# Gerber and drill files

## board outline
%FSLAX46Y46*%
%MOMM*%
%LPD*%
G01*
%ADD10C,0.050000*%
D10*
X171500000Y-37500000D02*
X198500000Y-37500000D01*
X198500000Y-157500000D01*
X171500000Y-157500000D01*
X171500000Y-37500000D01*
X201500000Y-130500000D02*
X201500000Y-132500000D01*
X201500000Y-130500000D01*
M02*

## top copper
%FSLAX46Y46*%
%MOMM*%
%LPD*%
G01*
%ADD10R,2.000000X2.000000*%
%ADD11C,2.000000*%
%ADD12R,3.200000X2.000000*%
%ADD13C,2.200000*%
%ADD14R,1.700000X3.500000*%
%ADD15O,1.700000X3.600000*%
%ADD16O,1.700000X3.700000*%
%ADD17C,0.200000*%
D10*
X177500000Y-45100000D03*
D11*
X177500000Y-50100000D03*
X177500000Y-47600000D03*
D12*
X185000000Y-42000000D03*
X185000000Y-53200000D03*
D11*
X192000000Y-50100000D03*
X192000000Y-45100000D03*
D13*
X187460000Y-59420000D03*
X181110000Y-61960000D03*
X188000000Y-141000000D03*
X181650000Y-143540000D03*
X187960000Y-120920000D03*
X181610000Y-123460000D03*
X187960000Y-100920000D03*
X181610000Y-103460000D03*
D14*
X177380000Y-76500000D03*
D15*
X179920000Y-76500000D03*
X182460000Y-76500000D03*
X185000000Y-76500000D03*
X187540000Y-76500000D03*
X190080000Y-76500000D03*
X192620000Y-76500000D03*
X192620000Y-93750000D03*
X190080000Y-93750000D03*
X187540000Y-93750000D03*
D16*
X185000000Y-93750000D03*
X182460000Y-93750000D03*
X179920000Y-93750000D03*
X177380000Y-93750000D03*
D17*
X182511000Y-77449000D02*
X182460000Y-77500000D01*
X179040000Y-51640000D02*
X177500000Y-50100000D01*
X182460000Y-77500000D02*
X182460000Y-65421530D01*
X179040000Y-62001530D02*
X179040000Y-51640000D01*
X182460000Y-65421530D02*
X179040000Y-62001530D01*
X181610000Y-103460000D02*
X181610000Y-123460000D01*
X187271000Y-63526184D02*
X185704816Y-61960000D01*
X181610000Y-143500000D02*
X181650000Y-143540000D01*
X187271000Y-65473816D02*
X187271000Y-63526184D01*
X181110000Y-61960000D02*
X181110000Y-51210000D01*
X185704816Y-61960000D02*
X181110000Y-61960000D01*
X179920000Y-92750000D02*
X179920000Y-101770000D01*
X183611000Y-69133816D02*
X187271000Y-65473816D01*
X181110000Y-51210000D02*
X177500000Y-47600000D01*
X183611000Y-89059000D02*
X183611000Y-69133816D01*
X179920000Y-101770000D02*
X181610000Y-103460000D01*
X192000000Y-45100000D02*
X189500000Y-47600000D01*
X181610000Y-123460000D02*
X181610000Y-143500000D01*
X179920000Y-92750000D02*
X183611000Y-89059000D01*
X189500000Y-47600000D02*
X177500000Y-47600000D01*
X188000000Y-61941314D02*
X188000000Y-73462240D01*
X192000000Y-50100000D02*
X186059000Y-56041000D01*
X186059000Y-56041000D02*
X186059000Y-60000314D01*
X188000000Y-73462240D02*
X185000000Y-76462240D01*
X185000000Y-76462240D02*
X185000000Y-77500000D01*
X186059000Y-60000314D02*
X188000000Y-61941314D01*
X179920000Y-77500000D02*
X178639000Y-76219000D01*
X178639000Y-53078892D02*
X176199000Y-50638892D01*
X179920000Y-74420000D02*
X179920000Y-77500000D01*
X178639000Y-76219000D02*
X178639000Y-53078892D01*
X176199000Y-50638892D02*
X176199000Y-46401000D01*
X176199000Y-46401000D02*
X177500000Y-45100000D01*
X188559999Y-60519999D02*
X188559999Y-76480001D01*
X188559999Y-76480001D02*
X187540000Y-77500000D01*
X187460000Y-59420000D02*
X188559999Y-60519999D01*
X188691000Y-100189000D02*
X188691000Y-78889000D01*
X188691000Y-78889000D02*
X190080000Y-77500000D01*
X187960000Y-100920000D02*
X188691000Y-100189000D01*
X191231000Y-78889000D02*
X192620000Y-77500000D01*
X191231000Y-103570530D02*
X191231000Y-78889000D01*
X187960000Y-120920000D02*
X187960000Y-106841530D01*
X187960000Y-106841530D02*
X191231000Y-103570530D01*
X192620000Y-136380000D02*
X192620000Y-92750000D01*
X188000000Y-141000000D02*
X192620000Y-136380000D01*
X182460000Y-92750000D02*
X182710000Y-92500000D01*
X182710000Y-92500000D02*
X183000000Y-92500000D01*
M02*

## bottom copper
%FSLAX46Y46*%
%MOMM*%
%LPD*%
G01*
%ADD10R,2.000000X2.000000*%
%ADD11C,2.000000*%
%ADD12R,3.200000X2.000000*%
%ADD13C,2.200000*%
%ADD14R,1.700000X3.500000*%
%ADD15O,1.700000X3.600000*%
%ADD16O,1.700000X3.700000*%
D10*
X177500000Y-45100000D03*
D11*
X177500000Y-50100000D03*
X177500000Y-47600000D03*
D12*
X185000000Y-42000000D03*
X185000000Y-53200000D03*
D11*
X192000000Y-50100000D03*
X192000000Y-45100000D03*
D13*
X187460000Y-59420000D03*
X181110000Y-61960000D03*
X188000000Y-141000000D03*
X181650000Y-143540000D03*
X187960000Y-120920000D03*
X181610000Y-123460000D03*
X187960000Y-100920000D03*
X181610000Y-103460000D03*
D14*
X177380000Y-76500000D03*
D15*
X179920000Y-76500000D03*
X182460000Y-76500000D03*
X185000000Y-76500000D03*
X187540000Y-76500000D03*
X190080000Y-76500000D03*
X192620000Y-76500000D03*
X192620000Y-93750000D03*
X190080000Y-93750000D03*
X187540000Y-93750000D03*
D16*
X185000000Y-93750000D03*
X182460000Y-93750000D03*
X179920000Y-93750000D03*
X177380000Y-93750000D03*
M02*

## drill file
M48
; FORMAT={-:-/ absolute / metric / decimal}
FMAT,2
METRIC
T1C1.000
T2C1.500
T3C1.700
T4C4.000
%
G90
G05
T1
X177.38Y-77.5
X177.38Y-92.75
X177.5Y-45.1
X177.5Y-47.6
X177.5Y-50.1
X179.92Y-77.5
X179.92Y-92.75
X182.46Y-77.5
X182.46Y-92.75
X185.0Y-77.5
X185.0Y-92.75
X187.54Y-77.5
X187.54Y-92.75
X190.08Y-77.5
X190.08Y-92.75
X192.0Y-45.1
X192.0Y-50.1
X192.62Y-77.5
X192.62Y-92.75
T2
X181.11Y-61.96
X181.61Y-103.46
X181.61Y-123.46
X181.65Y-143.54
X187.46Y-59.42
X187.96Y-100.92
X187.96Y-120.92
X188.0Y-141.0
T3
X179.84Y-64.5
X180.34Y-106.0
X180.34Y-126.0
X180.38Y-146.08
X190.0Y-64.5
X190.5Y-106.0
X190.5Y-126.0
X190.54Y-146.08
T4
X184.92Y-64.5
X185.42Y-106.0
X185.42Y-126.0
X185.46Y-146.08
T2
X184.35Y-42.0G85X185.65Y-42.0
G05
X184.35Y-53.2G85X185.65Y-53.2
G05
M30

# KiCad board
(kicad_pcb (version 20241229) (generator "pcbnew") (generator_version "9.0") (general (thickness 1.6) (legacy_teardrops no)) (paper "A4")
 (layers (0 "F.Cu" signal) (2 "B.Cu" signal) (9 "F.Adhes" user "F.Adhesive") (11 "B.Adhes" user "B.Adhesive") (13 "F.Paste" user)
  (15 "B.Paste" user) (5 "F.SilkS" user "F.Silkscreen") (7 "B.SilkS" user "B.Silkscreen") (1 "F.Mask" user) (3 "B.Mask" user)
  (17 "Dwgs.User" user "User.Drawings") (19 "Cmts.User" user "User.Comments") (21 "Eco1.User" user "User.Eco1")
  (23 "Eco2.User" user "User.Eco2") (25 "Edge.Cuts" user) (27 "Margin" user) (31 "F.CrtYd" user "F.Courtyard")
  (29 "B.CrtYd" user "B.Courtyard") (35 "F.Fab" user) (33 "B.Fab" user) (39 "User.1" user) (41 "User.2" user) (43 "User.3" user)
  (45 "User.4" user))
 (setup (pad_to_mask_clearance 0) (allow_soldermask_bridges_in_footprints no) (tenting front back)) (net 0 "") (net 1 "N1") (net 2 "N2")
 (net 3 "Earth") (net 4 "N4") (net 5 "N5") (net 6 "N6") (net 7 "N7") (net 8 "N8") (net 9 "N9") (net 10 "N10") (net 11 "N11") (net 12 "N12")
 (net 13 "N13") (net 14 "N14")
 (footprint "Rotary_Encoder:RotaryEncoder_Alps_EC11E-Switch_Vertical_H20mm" (layer "F.Cu") (at 177.5 45.1)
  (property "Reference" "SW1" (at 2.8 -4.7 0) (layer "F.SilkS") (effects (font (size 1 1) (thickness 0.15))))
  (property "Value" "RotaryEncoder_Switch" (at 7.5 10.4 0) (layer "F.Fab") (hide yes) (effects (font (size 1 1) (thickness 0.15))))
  (pad "A" thru_hole rect (at 0 0) (size 2 2) (drill 1) (layers "*.Cu" "*.Mask") (remove_unused_layers no) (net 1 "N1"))
  (pad "B" thru_hole circle (at 0 5) (size 2 2) (drill 1) (layers "*.Cu" "*.Mask") (remove_unused_layers no) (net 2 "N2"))
  (pad "C" thru_hole circle (at 0 2.5) (size 2 2) (drill 1) (layers "*.Cu" "*.Mask") (remove_unused_layers no) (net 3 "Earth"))
  (pad "MP" thru_hole rect (at 7.5 -3.1) (size 3.2 2) (drill oval 2.8 1.5) (layers "*.Cu" "*.Mask") (remove_unused_layers no))
  (pad "MP" thru_hole rect (at 7.5 8.1) (size 3.2 2) (drill oval 2.8 1.5) (layers "*.Cu" "*.Mask") (remove_unused_layers no))
  (pad "S1" thru_hole circle (at 14.5 5) (size 2 2) (drill 1) (layers "*.Cu" "*.Mask") (remove_unused_layers no) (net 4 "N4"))
  (pad "S2" thru_hole circle (at 14.5 0) (size 2 2) (drill 1) (layers "*.Cu" "*.Mask") (remove_unused_layers no) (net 3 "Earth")))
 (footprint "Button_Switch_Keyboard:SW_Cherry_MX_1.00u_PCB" (layer "F.Cu") (at 187.46 59.42)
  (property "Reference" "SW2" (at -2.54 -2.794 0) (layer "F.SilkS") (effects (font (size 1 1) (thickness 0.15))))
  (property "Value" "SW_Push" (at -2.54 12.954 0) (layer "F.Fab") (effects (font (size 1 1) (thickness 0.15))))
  (pad "" np_thru_hole circle (at -7.62 5.08) (size 1.7 1.7) (drill 1.7) (layers "*.Cu" "*.Mask"))
  (pad "" np_thru_hole circle (at -2.54 5.08) (size 4 4) (drill 4) (layers "*.Cu" "*.Mask"))
  (pad "" np_thru_hole circle (at 2.54 5.08) (size 1.7 1.7) (drill 1.7) (layers "*.Cu" "*.Mask"))
  (pad "1" thru_hole circle (at 0 0) (size 2.2 2.2) (drill 1.5) (layers "*.Cu" "*.Mask") (remove_unused_layers no) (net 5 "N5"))
  (pad "2" thru_hole circle (at -6.35 2.54) (size 2.2 2.2) (drill 1.5) (layers "*.Cu" "*.Mask") (remove_unused_layers no) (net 3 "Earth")))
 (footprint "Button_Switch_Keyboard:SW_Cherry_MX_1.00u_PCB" (layer "F.Cu") (at 188 141)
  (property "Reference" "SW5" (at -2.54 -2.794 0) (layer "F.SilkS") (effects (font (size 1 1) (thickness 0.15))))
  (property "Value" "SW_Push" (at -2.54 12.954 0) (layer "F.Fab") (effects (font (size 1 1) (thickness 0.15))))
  (pad "" np_thru_hole circle (at -7.62 5.08) (size 1.7 1.7) (drill 1.7) (layers "*.Cu" "*.Mask"))
  (pad "" np_thru_hole circle (at -2.54 5.08) (size 4 4) (drill 4) (layers "*.Cu" "*.Mask"))
  (pad "" np_thru_hole circle (at 2.54 5.08) (size 1.7 1.7) (drill 1.7) (layers "*.Cu" "*.Mask"))
  (pad "1" thru_hole circle (at 0 0) (size 2.2 2.2) (drill 1.5) (layers "*.Cu" "*.Mask") (remove_unused_layers no) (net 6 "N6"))
  (pad "2" thru_hole circle (at -6.35 2.54) (size 2.2 2.2) (drill 1.5) (layers "*.Cu" "*.Mask") (remove_unused_layers no) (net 3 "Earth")))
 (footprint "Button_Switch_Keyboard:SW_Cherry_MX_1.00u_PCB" (layer "F.Cu") (at 187.96 120.92)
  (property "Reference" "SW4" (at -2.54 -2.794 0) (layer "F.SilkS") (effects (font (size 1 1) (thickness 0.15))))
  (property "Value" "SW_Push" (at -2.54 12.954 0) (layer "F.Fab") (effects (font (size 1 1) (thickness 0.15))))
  (pad "" np_thru_hole circle (at -7.62 5.08) (size 1.7 1.7) (drill 1.7) (layers "*.Cu" "*.Mask"))
  (pad "" np_thru_hole circle (at -2.54 5.08) (size 4 4) (drill 4) (layers "*.Cu" "*.Mask"))
  (pad "" np_thru_hole circle (at 2.54 5.08) (size 1.7 1.7) (drill 1.7) (layers "*.Cu" "*.Mask"))
  (pad "1" thru_hole circle (at 0 0) (size 2.2 2.2) (drill 1.5) (layers "*.Cu" "*.Mask") (remove_unused_layers no) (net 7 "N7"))
  (pad "2" thru_hole circle (at -6.35 2.54) (size 2.2 2.2) (drill 1.5) (layers "*.Cu" "*.Mask") (remove_unused_layers no) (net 3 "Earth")))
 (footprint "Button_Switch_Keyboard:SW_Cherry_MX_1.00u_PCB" (layer "F.Cu") (at 187.96 100.92)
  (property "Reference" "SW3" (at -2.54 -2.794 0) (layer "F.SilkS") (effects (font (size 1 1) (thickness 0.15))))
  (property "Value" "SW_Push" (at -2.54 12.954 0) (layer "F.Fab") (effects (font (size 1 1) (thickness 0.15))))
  (pad "" np_thru_hole circle (at -7.62 5.08) (size 1.7 1.7) (drill 1.7) (layers "*.Cu" "*.Mask"))
  (pad "" np_thru_hole circle (at -2.54 5.08) (size 4 4) (drill 4) (layers "*.Cu" "*.Mask"))
  (pad "" np_thru_hole circle (at 2.54 5.08) (size 1.7 1.7) (drill 1.7) (layers "*.Cu" "*.Mask"))
  (pad "1" thru_hole circle (at 0 0) (size 2.2 2.2) (drill 1.5) (layers "*.Cu" "*.Mask") (remove_unused_layers no) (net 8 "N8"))
  (pad "2" thru_hole circle (at -6.35 2.54) (size 2.2 2.2) (drill 1.5) (layers "*.Cu" "*.Mask") (remove_unused_layers no) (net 3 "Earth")))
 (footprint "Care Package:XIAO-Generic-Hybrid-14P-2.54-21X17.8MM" (layer "B.Cu") (at 185 85.125 -90)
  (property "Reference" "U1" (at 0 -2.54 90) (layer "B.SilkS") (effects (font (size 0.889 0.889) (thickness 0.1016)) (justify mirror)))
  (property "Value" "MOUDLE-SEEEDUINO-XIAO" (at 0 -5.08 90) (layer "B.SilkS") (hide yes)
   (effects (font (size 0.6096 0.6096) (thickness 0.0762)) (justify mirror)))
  (pad "1" thru_hole rect (at -7.625 7.62 270) (size 3.5 1.7) (drill 1 (offset -1 0)) (layers "*.Cu" "*.Mask") (remove_unused_layers no)
   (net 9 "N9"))
  (pad "2" thru_hole oval (at -7.625 5.08 270) (size 3.6 1.7) (drill 1 (offset -1 0)) (layers "*.Cu" "*.Mask") (remove_unused_layers no)
   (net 1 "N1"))
  (pad "3" thru_hole oval (at -7.625 2.54 270) (size 3.6 1.7) (drill 1 (offset -1 0)) (layers "*.Cu" "*.Mask") (remove_unused_layers no)
   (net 2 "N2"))
  (pad "4" thru_hole oval (at -7.625 0 270) (size 3.6 1.7) (drill 1 (offset -1 0)) (layers "*.Cu" "*.Mask") (remove_unused_layers no)
   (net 4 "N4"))
  (pad "5" thru_hole oval (at -7.625 -2.54 270) (size 3.6 1.7) (drill 1 (offset -1 0)) (layers "*.Cu" "*.Mask") (remove_unused_layers no)
   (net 5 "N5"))
  (pad "6" thru_hole oval (at -7.625 -5.08 90) (size 3.6 1.7) (drill 1 (offset 1 0)) (layers "*.Cu" "*.Mask") (remove_unused_layers no)
   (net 8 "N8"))
  (pad "7" thru_hole oval (at -7.625 -7.62 270) (size 3.6 1.7) (drill 1 (offset -1 0)) (layers "*.Cu" "*.Mask") (remove_unused_layers no)
   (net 7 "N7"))
  (pad "8" thru_hole oval (at 7.625 -7.62 270) (size 3.6 1.7) (drill 1 (offset 1 0)) (layers "*.Cu" "*.Mask") (remove_unused_layers no)
   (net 6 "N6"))
  (pad "9" thru_hole oval (at 7.625 -5.08 270) (size 3.6 1.7) (drill 1 (offset 1 0)) (layers "*.Cu" "*.Mask") (remove_unused_layers no)
   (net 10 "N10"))
  (pad "10" thru_hole oval (at 7.625 -2.54 270) (size 3.6 1.7) (drill 1 (offset 1 0)) (layers "*.Cu" "*.Mask") (remove_unused_layers no)
   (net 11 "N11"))
  (pad "11" thru_hole oval (at 7.625 0 270) (size 3.7 1.7) (drill 1 (offset 1 0)) (layers "*.Cu" "*.Mask") (remove_unused_layers no)
   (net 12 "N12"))
  (pad "12" thru_hole oval (at 7.625 2.54 270) (size 3.7 1.7) (drill 1 (offset 1 0)) (layers "*.Cu" "*.Mask") (remove_unused_layers no)
   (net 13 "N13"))
  (pad "13" thru_hole oval (at 7.625 5.08 270) (size 3.7 1.7) (drill 1 (offset 1 0)) (layers "*.Cu" "*.Mask") (remove_unused_layers no)
   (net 3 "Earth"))
  (pad "14" thru_hole oval (at 7.625 7.62 270) (size 3.7 1.7) (drill 1 (offset 1 0)) (layers "*.Cu" "*.Mask") (remove_unused_layers no)
   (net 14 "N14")))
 (gr_rect (start 171.5 37.5) (end 198.5 157.5) (stroke (width 0.05) (type default)) (fill no) (layer "Edge.Cuts"))
 (gr_rect (start 201.5 130.5) (end 201.5 132.5) (stroke (width 0.05) (type default)) (fill no) (layer "Edge.Cuts"))
 (segment (start 182.511 77.449) (end 182.46 77.5) (width 0.2) (layer "F.Cu") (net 2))
 (segment (start 179.04 51.64) (end 177.5 50.1) (width 0.2) (layer "F.Cu") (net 2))
 (segment (start 182.46 77.5) (end 182.46 65.42153) (width 0.2) (layer "F.Cu") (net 2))
 (segment (start 179.04 62.00153) (end 179.04 51.64) (width 0.2) (layer "F.Cu") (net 2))
 (segment (start 182.46 65.42153) (end 179.04 62.00153) (width 0.2) (layer "F.Cu") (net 2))
 (segment (start 181.61 103.46) (end 181.61 123.46) (width 0.2) (layer "F.Cu") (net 3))
 (segment (start 187.271 63.526184) (end 185.704816 61.96) (width 0.2) (layer "F.Cu") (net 3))
 (segment (start 181.61 143.5) (end 181.65 143.54) (width 0.2) (layer "F.Cu") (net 3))
 (segment (start 187.271 65.473816) (end 187.271 63.526184) (width 0.2) (layer "F.Cu") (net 3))
 (segment (start 181.11 61.96) (end 181.11 51.21) (width 0.2) (layer "F.Cu") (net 3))
 (segment (start 185.704816 61.96) (end 181.11 61.96) (width 0.2) (layer "F.Cu") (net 3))
 (segment (start 179.92 92.75) (end 179.92 101.77) (width 0.2) (layer "F.Cu") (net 3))
 (segment (start 183.611 69.133816) (end 187.271 65.473816) (width 0.2) (layer "F.Cu") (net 3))
 (segment (start 181.11 51.21) (end 177.5 47.6) (width 0.2) (layer "F.Cu") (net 3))
 (segment (start 183.611 89.059) (end 183.611 69.133816) (width 0.2) (layer "F.Cu") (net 3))
 (segment (start 179.92 101.77) (end 181.61 103.46) (width 0.2) (layer "F.Cu") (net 3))
 (segment (start 192 45.1) (end 189.5 47.6) (width 0.2) (layer "F.Cu") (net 3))
 (segment (start 181.61 123.46) (end 181.61 143.5) (width 0.2) (layer "F.Cu") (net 3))
 (segment (start 179.92 92.75) (end 183.611 89.059) (width 0.2) (layer "F.Cu") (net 3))
 (segment (start 189.5 47.6) (end 177.5 47.6) (width 0.2) (layer "F.Cu") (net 3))
 (segment (start 188 61.941314) (end 188 73.46224) (width 0.2) (layer "F.Cu") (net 4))
 (segment (start 192 50.1) (end 186.059 56.041) (width 0.2) (layer "F.Cu") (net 4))
 (segment (start 186.059 56.041) (end 186.059 60.000314) (width 0.2) (layer "F.Cu") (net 4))
 (segment (start 188 73.46224) (end 185 76.46224) (width 0.2) (layer "F.Cu") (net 4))
 (segment (start 185 76.46224) (end 185 77.5) (width 0.2) (layer "F.Cu") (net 4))
 (segment (start 186.059 60.000314) (end 188 61.941314) (width 0.2) (layer "F.Cu") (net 4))
 (segment (start 179.92 77.5) (end 178.639 76.219) (width 0.2) (layer "F.Cu") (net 1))
 (segment (start 178.639 53.078892) (end 176.199 50.638892) (width 0.2) (layer "F.Cu") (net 1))
 (segment (start 179.92 74.42) (end 179.92 77.5) (width 0.2) (layer "F.Cu") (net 1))
 (segment (start 178.639 76.219) (end 178.639 53.078892) (width 0.2) (layer "F.Cu") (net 1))
 (segment (start 176.199 50.638892) (end 176.199 46.401) (width 0.2) (layer "F.Cu") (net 1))
 (segment (start 176.199 46.401) (end 177.5 45.1) (width 0.2) (layer "F.Cu") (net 1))
 (segment (start 188.559999 60.519999) (end 188.559999 76.480001) (width 0.2) (layer "F.Cu") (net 5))
 (segment (start 188.559999 76.480001) (end 187.54 77.5) (width 0.2) (layer "F.Cu") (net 5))
 (segment (start 187.46 59.42) (end 188.559999 60.519999) (width 0.2) (layer "F.Cu") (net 5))
 (segment (start 188.691 100.189) (end 188.691 78.889) (width 0.2) (layer "F.Cu") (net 8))
 (segment (start 188.691 78.889) (end 190.08 77.5) (width 0.2) (layer "F.Cu") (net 8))
 (segment (start 187.96 100.92) (end 188.691 100.189) (width 0.2) (layer "F.Cu") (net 8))
 (segment (start 191.231 78.889) (end 192.62 77.5) (width 0.2) (layer "F.Cu") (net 7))
 (segment (start 191.231 103.57053) (end 191.231 78.889) (width 0.2) (layer "F.Cu") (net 7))
 (segment (start 187.96 120.92) (end 187.96 106.84153) (width 0.2) (layer "F.Cu") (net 7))
 (segment (start 187.96 106.84153) (end 191.231 103.57053) (width 0.2) (layer "F.Cu") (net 7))
 (segment (start 192.62 136.38) (end 192.62 92.75) (width 0.2) (layer "F.Cu") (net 6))
 (segment (start 188 141) (end 192.62 136.38) (width 0.2) (layer "F.Cu") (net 6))
 (segment (start 182.46 92.75) (end 182.71 92.5) (width 0.2) (layer "F.Cu") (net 13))
 (segment (start 182.71 92.5) (end 183 92.5) (width 0.2) (layer "F.Cu") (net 13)))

